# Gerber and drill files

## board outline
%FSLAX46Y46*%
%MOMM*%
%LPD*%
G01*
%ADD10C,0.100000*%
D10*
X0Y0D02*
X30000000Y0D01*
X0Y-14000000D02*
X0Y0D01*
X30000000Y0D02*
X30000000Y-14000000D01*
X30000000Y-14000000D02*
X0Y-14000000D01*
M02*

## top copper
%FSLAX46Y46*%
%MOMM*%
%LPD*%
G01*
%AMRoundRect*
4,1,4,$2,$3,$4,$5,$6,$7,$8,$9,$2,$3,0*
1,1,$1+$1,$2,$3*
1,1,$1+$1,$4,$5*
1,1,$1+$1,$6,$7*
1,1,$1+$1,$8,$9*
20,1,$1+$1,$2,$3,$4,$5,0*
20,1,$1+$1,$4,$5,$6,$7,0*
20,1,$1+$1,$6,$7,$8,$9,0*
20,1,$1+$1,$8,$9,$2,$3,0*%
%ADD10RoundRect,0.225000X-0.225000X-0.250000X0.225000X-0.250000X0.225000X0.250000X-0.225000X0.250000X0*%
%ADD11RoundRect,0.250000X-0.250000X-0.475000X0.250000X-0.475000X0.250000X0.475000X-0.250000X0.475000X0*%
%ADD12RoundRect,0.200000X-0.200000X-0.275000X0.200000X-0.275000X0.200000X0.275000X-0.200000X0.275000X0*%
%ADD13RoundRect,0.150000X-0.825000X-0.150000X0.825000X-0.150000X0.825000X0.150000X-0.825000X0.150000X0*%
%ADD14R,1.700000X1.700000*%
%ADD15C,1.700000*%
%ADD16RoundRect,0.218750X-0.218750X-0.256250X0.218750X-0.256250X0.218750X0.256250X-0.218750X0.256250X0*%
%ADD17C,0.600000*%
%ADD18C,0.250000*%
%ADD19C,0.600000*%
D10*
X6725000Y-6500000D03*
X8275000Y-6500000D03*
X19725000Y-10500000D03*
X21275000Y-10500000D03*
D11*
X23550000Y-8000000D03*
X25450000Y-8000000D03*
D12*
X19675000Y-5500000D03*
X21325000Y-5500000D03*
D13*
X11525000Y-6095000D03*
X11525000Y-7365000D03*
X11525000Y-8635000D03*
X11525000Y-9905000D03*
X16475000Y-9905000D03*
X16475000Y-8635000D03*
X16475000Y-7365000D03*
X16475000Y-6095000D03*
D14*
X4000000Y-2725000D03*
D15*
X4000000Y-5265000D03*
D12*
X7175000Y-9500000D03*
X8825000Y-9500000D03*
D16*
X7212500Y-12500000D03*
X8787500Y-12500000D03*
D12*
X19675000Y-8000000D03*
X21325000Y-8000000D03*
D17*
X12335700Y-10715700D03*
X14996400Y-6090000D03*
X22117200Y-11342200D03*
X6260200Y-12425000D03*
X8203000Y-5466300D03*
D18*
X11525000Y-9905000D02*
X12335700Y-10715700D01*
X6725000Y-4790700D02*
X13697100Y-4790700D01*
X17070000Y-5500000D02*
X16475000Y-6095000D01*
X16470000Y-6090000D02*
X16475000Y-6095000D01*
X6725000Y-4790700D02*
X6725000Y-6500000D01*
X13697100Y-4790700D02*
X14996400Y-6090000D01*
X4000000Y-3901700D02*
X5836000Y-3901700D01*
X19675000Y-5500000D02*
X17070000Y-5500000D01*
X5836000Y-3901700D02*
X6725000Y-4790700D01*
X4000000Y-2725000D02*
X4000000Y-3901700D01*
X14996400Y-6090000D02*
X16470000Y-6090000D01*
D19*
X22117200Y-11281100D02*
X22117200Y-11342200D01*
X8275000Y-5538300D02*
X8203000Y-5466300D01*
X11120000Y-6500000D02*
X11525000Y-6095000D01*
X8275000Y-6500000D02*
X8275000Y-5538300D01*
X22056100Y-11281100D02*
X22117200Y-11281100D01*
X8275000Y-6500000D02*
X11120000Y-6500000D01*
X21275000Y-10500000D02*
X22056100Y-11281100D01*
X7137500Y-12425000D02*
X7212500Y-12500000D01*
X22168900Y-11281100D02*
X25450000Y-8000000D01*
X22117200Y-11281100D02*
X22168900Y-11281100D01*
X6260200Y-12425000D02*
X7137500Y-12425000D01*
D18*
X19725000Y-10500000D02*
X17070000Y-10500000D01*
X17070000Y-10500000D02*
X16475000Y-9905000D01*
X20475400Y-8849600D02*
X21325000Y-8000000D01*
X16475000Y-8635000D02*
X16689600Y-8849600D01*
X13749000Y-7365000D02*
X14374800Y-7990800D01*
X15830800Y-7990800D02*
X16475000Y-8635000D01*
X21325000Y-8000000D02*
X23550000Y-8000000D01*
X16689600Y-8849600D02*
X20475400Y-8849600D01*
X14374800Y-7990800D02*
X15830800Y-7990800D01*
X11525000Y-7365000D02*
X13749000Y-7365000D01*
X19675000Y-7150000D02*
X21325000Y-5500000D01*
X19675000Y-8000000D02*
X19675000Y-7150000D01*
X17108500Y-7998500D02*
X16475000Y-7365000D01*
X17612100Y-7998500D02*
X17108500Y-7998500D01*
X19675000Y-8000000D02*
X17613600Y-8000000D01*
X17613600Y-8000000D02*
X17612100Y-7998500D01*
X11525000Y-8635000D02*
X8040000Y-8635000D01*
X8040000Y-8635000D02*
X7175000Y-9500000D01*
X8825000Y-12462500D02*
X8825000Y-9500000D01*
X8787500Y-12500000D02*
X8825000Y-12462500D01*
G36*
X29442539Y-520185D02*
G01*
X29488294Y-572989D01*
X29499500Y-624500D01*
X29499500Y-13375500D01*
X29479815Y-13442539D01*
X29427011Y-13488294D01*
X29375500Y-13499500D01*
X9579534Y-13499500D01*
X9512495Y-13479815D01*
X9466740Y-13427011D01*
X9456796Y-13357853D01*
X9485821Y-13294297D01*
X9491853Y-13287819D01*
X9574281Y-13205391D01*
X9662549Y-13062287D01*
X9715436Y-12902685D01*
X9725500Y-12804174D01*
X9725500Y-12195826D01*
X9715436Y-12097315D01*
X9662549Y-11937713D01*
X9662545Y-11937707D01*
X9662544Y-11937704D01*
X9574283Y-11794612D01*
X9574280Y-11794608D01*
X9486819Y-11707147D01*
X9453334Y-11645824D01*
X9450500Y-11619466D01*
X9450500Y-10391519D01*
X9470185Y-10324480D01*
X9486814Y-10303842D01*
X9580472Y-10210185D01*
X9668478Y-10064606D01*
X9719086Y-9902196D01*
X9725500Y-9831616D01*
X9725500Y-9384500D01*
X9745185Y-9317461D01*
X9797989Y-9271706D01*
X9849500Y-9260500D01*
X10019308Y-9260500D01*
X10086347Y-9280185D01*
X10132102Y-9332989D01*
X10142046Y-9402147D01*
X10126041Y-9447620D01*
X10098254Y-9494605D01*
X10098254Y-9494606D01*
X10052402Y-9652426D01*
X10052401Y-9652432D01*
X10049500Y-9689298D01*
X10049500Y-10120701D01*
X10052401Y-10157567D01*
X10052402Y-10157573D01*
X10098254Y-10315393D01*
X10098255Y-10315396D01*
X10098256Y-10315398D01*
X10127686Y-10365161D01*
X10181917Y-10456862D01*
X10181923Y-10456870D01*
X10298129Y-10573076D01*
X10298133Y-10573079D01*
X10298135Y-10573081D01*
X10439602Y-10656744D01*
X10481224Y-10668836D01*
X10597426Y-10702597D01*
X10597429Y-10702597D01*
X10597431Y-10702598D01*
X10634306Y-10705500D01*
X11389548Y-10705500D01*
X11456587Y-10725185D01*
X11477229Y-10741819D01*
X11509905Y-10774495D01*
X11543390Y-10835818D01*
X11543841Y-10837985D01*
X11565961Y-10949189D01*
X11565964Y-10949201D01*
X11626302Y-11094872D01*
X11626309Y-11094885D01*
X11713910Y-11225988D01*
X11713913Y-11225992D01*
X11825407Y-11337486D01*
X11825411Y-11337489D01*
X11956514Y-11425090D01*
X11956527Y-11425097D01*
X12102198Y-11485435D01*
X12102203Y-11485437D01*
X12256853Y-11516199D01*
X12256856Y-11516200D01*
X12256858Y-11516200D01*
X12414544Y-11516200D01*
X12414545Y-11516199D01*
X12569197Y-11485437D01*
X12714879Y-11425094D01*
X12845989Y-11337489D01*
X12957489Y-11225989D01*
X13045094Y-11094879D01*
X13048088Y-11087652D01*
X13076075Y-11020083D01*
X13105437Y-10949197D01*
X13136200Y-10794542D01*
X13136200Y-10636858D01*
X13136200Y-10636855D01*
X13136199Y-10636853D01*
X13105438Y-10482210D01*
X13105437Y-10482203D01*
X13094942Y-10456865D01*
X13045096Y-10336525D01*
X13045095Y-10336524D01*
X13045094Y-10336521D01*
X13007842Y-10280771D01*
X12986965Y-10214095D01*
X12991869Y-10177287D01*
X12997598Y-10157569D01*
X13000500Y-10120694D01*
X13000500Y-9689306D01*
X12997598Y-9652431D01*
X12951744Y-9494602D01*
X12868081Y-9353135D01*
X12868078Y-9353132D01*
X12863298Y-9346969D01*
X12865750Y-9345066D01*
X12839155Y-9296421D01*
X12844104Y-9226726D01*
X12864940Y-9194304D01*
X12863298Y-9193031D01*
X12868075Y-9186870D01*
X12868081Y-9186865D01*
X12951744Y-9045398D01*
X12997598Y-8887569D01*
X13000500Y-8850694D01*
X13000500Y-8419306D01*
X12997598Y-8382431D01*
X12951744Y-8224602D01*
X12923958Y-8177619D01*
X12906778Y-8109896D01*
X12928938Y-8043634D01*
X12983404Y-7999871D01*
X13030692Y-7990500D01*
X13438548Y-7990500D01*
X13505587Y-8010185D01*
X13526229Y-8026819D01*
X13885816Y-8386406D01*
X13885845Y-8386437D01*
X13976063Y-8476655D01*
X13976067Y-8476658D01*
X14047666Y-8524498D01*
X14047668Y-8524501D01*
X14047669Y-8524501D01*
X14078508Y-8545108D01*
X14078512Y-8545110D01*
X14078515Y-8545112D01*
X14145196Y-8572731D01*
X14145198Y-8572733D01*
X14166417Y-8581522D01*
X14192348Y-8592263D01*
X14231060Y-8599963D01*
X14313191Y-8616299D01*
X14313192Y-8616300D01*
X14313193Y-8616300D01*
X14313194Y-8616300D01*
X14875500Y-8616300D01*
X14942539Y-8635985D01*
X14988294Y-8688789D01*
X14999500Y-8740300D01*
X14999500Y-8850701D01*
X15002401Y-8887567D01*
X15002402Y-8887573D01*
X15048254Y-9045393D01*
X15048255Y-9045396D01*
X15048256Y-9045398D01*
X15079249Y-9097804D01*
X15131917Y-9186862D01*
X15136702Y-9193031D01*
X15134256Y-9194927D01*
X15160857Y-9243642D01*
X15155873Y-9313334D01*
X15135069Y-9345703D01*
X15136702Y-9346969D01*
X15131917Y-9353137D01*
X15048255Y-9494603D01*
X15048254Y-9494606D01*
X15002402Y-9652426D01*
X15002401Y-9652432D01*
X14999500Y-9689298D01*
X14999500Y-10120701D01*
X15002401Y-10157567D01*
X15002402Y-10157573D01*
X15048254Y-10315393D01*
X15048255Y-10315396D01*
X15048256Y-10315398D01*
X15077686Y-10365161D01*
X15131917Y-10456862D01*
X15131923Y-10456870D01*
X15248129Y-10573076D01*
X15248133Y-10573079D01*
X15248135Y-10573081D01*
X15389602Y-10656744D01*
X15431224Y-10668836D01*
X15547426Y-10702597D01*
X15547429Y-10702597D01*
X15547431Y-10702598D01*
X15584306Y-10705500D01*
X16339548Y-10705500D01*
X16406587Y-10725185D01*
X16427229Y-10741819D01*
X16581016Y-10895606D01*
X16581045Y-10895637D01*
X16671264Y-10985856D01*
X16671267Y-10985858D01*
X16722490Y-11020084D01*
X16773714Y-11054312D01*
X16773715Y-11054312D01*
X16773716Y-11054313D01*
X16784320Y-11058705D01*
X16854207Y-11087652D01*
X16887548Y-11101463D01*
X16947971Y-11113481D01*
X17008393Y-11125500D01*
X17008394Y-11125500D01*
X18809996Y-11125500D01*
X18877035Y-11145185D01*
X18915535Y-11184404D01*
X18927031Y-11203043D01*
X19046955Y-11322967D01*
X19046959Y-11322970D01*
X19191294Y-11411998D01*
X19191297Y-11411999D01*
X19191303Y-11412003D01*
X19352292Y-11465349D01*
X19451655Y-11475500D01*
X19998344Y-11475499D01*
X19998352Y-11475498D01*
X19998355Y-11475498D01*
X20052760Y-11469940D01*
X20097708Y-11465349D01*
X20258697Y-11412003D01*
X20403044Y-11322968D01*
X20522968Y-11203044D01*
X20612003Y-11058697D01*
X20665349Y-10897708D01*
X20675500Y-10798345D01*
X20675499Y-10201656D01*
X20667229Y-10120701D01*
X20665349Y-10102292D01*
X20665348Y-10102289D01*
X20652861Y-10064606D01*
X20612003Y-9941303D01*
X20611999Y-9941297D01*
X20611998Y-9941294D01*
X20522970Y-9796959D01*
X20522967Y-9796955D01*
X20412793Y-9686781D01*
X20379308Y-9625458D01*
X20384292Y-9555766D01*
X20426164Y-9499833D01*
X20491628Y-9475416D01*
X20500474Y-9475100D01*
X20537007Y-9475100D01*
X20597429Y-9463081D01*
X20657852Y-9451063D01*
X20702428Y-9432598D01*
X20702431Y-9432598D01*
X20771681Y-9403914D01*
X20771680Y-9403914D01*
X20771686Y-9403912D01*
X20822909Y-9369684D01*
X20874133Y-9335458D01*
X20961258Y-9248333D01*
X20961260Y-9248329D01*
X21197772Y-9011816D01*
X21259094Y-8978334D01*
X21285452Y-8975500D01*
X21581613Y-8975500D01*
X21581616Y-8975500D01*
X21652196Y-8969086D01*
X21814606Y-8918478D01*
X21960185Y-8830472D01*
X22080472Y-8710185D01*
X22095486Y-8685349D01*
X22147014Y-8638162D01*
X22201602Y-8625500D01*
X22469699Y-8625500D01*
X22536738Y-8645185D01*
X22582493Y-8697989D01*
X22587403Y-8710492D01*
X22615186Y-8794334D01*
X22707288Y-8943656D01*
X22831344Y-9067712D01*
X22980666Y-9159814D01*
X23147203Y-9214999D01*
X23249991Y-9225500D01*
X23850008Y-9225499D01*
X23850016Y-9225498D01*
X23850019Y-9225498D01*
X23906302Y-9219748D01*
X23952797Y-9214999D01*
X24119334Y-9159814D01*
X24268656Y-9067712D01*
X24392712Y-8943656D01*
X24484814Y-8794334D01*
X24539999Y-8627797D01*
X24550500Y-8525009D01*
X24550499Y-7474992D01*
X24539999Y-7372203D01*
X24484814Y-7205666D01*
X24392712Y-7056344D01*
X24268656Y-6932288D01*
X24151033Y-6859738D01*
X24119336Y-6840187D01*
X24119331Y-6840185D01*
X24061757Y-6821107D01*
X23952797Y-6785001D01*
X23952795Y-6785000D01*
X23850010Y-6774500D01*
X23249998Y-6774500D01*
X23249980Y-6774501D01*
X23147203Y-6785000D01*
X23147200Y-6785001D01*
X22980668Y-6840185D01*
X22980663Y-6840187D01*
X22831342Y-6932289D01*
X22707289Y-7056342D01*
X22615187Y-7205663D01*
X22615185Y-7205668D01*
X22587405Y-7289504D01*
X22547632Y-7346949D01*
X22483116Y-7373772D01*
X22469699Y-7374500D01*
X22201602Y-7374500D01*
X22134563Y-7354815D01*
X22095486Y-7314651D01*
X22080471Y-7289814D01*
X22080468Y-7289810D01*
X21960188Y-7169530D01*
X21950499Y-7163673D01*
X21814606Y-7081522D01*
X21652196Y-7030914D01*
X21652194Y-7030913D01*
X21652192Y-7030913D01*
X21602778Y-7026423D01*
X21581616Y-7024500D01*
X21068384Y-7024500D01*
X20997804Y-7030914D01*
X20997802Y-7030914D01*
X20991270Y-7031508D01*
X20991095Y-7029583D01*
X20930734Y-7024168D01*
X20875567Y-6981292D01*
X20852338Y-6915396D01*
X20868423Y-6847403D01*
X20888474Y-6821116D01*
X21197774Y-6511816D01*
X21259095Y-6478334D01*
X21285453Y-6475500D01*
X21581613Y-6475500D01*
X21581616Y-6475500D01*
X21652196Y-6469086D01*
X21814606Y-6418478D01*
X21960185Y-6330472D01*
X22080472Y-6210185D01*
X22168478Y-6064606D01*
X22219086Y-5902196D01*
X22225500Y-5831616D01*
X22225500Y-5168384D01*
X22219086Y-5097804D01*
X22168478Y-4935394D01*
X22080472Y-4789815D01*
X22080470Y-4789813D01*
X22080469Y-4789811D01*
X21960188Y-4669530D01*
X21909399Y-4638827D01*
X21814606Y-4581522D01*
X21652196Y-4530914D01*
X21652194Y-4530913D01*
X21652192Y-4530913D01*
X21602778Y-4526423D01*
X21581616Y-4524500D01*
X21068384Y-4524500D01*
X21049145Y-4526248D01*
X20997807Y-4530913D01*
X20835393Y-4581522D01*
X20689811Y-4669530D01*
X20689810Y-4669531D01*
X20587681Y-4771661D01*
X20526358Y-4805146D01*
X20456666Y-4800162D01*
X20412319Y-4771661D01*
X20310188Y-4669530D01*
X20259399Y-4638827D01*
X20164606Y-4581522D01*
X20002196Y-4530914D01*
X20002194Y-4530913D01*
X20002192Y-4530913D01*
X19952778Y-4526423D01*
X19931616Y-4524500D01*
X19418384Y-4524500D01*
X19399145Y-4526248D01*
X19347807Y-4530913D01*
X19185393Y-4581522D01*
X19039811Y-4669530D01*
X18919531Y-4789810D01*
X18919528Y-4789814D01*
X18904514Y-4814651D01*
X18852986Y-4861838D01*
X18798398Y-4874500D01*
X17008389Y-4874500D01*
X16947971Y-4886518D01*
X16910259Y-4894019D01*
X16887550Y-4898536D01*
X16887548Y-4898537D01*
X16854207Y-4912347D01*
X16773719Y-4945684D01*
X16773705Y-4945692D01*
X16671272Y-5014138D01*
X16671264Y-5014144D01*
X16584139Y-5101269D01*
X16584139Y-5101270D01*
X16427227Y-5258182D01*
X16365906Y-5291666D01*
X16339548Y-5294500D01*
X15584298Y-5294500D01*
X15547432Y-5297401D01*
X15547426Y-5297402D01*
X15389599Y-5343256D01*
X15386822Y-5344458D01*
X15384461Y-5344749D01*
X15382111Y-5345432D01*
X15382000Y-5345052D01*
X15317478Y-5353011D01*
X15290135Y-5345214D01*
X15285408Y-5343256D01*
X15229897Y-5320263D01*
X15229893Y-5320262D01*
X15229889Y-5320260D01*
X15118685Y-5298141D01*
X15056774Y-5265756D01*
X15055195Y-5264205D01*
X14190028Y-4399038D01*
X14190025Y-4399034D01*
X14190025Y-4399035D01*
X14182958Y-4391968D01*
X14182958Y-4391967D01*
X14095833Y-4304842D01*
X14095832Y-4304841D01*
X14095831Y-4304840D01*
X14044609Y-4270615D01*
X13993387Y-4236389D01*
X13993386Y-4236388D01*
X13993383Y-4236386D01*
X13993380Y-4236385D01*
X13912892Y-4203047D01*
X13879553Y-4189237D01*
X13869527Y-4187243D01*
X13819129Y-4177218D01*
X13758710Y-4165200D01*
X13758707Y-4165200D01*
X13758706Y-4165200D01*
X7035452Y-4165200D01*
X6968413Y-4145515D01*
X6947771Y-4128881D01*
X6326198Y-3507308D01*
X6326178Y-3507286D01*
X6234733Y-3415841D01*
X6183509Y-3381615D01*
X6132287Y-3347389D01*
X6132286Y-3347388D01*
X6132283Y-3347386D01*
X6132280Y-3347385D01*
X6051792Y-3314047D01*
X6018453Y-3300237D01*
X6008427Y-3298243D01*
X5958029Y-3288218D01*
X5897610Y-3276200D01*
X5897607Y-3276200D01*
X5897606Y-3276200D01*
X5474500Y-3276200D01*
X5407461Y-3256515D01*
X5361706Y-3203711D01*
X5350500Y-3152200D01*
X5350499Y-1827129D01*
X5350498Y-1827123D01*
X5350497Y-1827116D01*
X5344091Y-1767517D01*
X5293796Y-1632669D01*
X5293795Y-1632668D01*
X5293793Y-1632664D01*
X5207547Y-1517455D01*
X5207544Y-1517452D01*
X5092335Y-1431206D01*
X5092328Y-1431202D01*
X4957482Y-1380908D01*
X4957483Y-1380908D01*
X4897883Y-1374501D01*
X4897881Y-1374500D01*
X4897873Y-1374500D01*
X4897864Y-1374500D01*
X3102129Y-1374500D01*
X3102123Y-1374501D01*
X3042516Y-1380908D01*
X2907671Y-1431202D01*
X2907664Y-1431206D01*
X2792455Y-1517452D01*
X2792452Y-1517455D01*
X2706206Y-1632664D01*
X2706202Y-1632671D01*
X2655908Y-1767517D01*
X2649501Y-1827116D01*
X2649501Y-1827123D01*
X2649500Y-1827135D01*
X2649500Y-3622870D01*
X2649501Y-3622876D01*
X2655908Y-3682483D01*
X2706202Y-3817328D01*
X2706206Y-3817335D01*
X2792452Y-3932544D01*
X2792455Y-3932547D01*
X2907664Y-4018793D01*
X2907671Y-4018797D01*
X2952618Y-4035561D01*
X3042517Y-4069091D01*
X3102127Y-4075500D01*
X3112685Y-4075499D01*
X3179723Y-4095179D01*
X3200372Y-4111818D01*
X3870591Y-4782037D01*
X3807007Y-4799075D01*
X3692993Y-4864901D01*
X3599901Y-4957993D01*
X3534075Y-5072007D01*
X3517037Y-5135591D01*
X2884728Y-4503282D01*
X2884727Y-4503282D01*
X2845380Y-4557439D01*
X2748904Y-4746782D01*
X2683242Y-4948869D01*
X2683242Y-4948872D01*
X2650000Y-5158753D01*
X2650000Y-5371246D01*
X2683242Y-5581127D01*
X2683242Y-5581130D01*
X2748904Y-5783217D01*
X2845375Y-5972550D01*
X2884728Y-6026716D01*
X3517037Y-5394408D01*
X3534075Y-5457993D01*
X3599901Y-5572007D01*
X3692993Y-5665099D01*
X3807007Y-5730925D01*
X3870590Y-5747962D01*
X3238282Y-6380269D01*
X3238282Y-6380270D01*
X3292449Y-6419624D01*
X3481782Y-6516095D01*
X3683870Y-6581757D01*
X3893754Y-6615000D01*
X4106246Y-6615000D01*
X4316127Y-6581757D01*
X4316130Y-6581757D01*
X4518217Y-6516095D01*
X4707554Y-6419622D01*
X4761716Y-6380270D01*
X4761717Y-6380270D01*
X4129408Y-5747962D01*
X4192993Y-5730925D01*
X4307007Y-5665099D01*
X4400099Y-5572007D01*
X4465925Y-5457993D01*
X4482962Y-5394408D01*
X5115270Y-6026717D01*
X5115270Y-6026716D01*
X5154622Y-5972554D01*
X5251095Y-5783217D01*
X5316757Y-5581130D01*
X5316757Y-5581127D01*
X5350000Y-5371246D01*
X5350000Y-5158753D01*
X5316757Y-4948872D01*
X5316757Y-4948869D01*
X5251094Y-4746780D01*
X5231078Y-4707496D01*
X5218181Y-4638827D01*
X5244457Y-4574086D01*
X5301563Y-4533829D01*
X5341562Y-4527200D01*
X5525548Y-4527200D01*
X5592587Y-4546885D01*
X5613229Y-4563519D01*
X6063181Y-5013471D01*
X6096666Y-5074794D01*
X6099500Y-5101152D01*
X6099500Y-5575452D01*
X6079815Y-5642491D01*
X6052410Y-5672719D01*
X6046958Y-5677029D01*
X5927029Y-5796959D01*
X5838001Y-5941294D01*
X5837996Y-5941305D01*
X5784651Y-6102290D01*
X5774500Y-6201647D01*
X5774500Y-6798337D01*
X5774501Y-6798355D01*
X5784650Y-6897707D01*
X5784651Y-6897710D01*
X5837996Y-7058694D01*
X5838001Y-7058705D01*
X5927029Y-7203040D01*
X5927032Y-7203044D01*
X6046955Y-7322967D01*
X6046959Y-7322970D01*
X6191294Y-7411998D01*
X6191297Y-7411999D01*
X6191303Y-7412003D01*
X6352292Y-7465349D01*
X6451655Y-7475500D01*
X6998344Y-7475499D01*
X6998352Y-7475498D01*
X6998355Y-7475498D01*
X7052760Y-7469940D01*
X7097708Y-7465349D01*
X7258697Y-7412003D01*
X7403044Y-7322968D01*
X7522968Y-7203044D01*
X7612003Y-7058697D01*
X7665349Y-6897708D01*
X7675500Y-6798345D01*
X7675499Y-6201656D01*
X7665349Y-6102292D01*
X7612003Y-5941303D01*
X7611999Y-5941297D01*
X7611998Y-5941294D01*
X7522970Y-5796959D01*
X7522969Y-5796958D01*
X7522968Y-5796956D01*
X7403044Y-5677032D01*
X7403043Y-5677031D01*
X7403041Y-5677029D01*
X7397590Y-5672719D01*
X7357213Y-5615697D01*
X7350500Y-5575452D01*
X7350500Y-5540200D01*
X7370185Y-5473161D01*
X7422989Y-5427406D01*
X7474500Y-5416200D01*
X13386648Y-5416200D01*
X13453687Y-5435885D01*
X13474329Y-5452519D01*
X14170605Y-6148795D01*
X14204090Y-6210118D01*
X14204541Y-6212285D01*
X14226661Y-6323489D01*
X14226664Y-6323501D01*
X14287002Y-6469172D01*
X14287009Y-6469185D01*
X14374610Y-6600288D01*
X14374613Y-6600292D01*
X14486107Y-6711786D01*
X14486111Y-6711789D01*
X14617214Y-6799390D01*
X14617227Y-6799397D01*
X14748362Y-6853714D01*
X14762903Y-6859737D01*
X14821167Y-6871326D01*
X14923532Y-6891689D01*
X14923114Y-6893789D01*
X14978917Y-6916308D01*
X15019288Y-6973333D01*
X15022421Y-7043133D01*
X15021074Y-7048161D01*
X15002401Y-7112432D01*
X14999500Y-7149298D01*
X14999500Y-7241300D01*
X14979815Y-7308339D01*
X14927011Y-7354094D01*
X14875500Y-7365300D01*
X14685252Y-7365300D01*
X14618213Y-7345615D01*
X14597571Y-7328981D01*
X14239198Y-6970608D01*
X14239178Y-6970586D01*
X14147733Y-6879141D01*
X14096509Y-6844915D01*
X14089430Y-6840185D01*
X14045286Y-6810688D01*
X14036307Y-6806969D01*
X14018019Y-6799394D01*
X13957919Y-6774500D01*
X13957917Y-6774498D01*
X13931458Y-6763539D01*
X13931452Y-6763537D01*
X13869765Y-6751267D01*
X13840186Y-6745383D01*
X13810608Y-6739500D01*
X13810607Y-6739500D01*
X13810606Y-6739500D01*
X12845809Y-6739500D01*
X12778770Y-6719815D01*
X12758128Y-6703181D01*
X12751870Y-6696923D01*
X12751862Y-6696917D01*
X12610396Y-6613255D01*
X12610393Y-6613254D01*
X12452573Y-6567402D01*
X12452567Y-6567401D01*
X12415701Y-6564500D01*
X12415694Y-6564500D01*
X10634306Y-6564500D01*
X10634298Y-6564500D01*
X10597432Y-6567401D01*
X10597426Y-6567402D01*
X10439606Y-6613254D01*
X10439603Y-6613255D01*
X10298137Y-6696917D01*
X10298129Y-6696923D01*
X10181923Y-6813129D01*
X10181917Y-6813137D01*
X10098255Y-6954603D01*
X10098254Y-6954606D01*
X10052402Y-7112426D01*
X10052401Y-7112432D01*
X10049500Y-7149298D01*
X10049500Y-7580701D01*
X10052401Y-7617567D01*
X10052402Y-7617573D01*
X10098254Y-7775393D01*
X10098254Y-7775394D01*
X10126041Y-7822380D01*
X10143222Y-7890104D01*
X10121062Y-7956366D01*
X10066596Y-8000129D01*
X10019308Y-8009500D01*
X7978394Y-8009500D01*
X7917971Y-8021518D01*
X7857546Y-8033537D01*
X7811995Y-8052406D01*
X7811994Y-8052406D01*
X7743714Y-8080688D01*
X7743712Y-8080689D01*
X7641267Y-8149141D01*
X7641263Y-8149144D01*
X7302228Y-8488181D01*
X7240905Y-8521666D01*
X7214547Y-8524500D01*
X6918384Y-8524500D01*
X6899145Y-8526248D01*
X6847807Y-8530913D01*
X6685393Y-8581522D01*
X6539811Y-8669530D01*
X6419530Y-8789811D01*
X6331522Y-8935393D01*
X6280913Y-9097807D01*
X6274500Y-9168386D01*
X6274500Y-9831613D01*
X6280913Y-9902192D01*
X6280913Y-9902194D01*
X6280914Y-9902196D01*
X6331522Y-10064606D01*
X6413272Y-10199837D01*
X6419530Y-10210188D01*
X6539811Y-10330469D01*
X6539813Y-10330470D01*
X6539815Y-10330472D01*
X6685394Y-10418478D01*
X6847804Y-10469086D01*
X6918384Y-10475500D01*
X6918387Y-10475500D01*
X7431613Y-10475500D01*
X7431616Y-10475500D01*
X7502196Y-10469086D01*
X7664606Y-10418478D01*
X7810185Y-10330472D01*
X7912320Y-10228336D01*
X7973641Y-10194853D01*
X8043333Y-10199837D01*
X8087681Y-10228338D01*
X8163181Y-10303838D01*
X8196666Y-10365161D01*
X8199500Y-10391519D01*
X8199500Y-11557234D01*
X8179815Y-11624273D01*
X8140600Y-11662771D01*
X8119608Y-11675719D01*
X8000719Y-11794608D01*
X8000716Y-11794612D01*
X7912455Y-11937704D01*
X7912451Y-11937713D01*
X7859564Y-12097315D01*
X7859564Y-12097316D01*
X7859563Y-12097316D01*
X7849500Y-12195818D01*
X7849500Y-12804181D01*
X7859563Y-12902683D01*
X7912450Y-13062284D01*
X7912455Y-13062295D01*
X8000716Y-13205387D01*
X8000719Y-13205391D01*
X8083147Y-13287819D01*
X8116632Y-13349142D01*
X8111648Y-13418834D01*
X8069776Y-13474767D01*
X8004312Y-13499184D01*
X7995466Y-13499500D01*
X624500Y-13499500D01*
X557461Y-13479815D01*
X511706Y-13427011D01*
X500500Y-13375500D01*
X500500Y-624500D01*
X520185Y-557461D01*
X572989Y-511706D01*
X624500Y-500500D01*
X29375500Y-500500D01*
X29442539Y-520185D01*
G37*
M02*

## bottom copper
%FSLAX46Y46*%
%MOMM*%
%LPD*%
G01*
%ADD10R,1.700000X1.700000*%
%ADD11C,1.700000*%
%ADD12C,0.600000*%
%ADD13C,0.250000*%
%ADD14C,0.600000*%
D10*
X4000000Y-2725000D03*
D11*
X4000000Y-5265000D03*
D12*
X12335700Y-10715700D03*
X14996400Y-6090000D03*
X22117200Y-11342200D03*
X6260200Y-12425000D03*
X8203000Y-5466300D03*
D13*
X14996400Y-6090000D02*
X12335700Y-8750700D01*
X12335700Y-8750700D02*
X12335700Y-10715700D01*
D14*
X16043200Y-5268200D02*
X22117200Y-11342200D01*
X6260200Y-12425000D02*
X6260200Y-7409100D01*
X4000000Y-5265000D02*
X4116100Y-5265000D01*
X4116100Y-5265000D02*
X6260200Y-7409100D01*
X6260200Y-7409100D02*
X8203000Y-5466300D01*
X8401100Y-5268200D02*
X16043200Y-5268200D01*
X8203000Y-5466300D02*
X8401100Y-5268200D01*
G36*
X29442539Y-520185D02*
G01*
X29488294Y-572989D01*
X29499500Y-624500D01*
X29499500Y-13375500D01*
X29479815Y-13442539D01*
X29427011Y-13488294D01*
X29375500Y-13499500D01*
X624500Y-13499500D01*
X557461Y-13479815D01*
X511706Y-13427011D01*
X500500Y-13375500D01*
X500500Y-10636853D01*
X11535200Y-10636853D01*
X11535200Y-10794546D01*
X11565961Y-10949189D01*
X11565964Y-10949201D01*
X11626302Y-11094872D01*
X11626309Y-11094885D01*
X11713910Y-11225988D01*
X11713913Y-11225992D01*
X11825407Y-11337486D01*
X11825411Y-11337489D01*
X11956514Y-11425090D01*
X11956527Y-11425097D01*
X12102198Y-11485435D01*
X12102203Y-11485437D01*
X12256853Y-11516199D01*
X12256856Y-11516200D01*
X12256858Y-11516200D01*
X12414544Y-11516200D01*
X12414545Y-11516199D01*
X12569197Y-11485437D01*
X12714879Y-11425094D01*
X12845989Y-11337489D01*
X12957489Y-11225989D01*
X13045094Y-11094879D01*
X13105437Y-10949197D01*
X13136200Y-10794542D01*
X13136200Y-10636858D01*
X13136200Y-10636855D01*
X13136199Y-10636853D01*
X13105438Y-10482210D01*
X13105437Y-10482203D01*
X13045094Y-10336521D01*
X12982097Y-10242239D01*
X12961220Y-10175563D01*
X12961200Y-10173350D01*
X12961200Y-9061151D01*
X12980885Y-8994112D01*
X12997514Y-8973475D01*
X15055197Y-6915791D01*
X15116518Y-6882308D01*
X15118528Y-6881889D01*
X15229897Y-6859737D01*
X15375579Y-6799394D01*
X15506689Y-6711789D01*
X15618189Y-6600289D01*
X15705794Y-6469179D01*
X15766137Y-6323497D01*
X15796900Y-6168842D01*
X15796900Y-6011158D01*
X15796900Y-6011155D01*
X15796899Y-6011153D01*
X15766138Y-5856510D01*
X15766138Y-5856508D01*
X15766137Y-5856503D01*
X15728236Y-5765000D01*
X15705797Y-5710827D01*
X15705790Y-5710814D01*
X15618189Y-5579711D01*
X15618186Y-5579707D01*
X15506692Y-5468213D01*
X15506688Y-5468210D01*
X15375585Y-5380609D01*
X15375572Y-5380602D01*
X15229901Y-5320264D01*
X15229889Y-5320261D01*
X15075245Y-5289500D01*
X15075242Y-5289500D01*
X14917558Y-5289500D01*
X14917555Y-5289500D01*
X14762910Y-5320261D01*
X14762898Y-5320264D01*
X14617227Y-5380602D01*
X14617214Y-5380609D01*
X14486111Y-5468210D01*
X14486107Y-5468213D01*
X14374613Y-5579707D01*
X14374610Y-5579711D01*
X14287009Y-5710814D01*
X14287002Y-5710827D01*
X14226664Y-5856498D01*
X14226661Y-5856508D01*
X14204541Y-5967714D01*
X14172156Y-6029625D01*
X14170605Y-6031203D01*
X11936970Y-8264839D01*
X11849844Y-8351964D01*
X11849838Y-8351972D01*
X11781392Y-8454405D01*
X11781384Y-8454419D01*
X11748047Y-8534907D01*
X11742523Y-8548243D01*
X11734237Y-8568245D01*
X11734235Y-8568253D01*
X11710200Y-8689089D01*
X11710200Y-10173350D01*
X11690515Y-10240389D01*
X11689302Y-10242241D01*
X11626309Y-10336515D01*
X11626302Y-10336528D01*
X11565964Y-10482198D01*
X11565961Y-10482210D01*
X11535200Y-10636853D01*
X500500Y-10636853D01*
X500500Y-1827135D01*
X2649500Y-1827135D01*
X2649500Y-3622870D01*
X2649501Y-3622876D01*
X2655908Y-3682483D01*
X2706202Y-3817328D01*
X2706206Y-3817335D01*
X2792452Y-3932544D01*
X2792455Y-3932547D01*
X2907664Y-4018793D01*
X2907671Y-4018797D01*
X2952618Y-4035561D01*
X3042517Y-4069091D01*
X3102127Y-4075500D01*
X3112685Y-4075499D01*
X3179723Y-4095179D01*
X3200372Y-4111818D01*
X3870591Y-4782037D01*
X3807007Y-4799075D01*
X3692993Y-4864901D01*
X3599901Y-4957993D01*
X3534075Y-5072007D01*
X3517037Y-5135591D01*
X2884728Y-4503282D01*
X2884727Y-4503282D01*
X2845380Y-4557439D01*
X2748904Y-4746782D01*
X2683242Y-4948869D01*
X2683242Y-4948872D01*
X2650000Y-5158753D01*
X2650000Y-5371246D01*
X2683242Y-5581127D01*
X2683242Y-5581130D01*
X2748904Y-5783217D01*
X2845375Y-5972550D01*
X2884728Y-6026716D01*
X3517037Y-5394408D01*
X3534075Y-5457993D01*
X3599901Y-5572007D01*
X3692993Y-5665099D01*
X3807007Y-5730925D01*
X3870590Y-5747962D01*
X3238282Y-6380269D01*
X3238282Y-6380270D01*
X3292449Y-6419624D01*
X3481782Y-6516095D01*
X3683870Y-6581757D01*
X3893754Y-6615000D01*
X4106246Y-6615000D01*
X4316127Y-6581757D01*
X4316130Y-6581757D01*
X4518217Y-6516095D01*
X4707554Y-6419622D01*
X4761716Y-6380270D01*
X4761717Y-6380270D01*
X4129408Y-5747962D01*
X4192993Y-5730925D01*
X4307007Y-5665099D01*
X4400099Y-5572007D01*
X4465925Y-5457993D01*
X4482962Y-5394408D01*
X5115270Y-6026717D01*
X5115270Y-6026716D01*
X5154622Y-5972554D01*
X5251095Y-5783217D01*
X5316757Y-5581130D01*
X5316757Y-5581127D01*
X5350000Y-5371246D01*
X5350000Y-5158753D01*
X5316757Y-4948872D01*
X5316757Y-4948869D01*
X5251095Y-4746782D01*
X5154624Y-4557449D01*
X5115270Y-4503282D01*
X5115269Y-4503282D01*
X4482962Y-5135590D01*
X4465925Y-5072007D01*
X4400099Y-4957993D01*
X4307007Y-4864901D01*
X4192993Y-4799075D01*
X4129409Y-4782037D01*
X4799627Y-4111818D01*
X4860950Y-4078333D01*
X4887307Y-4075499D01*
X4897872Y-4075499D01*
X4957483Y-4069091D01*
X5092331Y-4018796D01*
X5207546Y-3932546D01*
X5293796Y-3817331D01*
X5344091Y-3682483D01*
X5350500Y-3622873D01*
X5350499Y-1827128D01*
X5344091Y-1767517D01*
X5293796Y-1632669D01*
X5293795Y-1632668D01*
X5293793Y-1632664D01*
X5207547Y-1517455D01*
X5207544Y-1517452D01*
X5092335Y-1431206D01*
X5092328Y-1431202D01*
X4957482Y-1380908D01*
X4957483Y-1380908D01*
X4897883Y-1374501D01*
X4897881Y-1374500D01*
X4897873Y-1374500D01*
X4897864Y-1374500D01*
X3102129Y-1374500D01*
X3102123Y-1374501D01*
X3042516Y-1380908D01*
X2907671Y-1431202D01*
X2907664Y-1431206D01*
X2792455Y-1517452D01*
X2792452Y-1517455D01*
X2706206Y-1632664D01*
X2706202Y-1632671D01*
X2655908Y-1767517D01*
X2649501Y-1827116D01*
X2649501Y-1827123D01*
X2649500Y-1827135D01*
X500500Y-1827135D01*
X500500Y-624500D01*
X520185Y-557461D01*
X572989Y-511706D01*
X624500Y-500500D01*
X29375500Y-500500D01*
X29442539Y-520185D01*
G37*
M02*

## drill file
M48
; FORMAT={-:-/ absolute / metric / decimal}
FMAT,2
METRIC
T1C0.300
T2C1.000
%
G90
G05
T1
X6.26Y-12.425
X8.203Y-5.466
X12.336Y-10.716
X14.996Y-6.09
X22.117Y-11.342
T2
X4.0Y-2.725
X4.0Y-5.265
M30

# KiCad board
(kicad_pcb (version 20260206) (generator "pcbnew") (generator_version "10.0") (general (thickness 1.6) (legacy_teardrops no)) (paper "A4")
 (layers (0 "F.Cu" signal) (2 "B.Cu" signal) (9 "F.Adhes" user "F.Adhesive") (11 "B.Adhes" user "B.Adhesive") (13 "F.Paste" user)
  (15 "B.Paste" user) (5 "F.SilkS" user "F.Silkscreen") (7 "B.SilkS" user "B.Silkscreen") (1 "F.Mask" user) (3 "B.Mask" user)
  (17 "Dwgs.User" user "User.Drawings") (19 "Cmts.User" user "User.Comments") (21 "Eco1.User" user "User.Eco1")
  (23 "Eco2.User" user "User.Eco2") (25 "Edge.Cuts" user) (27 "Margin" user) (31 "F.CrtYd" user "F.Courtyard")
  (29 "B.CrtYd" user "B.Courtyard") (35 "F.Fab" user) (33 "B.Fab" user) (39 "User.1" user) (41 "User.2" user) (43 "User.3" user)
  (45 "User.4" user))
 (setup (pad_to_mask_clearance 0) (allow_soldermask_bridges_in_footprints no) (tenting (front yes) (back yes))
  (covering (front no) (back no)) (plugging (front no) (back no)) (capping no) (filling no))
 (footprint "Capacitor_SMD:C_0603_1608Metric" (layer "F.Cu") (at 7.5 6.5)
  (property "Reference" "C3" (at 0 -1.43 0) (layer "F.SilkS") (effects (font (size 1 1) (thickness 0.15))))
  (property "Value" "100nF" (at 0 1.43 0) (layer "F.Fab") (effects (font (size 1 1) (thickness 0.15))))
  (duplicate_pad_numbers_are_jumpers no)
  (pad "1" smd roundrect (at -0.775 0) (size 0.9 0.95) (layers "F.Cu" "F.Mask" "F.Paste") (roundrect_rratio 0.25) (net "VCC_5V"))
  (pad "2" smd roundrect (at 0.775 0) (size 0.9 0.95) (layers "F.Cu" "F.Mask" "F.Paste") (roundrect_rratio 0.25) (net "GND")
   (zone_connect 2)))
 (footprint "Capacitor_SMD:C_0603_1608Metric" (layer "F.Cu") (at 20.5 10.5)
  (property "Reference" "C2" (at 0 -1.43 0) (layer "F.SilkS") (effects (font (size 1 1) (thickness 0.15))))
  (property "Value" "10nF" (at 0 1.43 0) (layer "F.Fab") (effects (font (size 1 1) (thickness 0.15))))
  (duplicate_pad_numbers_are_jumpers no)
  (pad "1" smd roundrect (at -0.775 0) (size 0.9 0.95) (layers "F.Cu" "F.Mask" "F.Paste") (roundrect_rratio 0.25) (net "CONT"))
  (pad "2" smd roundrect (at 0.775 0) (size 0.9 0.95) (layers "F.Cu" "F.Mask" "F.Paste") (roundrect_rratio 0.25) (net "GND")
   (zone_connect 2)))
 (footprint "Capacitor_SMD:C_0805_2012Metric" (layer "F.Cu") (at 24.5 8)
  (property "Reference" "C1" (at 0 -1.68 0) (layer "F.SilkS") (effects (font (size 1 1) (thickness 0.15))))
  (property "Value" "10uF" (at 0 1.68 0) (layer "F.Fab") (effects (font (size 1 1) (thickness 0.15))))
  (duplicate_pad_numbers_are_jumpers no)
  (pad "1" smd roundrect (at -0.95 0) (size 1 1.45) (layers "F.Cu" "F.Mask" "F.Paste") (roundrect_rratio 0.25) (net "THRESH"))
  (pad "2" smd roundrect (at 0.95 0) (size 1 1.45) (layers "F.Cu" "F.Mask" "F.Paste") (roundrect_rratio 0.25) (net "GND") (zone_connect 2)))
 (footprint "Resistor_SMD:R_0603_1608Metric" (layer "F.Cu") (at 20.5 5.5)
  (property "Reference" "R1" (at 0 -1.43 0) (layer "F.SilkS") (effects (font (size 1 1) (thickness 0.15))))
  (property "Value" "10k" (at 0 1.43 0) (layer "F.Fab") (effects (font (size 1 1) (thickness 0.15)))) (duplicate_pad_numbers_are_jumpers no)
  (pad "1" smd roundrect (at -0.825 0) (size 0.8 0.95) (layers "F.Cu" "F.Mask" "F.Paste") (roundrect_rratio 0.25) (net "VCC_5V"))
  (pad "2" smd roundrect (at 0.825 0) (size 0.8 0.95) (layers "F.Cu" "F.Mask" "F.Paste") (roundrect_rratio 0.25) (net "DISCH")))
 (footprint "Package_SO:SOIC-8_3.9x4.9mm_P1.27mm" (layer "F.Cu") (at 14 8)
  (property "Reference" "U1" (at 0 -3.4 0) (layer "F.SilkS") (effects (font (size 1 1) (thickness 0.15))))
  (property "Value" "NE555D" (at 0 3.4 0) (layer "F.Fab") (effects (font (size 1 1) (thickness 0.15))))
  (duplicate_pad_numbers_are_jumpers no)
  (pad "1" smd roundrect (at -2.475 -1.905) (size 1.95 0.6) (layers "F.Cu" "F.Mask" "F.Paste") (roundrect_rratio 0.25) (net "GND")
   (zone_connect 2))
  (pad "2" smd roundrect (at -2.475 -0.635) (size 1.95 0.6) (layers "F.Cu" "F.Mask" "F.Paste") (roundrect_rratio 0.25) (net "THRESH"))
  (pad "3" smd roundrect (at -2.475 0.635) (size 1.95 0.6) (layers "F.Cu" "F.Mask" "F.Paste") (roundrect_rratio 0.25) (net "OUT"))
  (pad "4" smd roundrect (at -2.475 1.905) (size 1.95 0.6) (layers "F.Cu" "F.Mask" "F.Paste") (roundrect_rratio 0.25) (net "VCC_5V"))
  (pad "5" smd roundrect (at 2.475 1.905) (size 1.95 0.6) (layers "F.Cu" "F.Mask" "F.Paste") (roundrect_rratio 0.25) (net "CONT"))
  (pad "6" smd roundrect (at 2.475 0.635) (size 1.95 0.6) (layers "F.Cu" "F.Mask" "F.Paste") (roundrect_rratio 0.25) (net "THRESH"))
  (pad "7" smd roundrect (at 2.475 -0.635) (size 1.95 0.6) (layers "F.Cu" "F.Mask" "F.Paste") (roundrect_rratio 0.25) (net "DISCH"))
  (pad "8" smd roundrect (at 2.475 -1.905) (size 1.95 0.6) (layers "F.Cu" "F.Mask" "F.Paste") (roundrect_rratio 0.25) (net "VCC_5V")))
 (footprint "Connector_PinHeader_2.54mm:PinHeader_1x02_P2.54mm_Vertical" (layer "F.Cu") (at 4 2.725)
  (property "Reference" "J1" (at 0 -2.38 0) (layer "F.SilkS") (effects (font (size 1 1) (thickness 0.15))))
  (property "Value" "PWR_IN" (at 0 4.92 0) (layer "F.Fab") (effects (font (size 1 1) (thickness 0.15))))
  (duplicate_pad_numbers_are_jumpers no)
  (pad "1" thru_hole rect (at 0 0) (size 1.7 1.7) (drill 1) (layers "*.Cu" "*.Mask") (remove_unused_layers no) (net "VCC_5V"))
  (pad "2" thru_hole circle (at 0 2.54) (size 1.7 1.7) (drill 1) (layers "*.Cu" "*.Mask") (remove_unused_layers no) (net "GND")))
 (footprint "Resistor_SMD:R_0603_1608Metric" (layer "F.Cu") (at 8 9.5)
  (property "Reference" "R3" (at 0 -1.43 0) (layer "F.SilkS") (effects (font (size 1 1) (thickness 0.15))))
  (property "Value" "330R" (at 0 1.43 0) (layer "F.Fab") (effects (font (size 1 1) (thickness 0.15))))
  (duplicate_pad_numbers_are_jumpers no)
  (pad "1" smd roundrect (at -0.825 0) (size 0.8 0.95) (layers "F.Cu" "F.Mask" "F.Paste") (roundrect_rratio 0.25) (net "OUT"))
  (pad "2" smd roundrect (at 0.825 0) (size 0.8 0.95) (layers "F.Cu" "F.Mask" "F.Paste") (roundrect_rratio 0.25) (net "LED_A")))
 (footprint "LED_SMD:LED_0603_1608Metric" (layer "F.Cu") (at 8 12.5)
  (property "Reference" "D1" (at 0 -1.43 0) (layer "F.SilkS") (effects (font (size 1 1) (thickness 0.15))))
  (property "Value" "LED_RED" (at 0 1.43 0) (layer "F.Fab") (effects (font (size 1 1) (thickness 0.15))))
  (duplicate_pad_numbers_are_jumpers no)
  (pad "1" smd roundrect (at -0.7875 0) (size 0.875 0.95) (layers "F.Cu" "F.Mask" "F.Paste") (roundrect_rratio 0.25) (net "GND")
   (zone_connect 2))
  (pad "2" smd roundrect (at 0.7875 0) (size 0.875 0.95) (layers "F.Cu" "F.Mask" "F.Paste") (roundrect_rratio 0.25) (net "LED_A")))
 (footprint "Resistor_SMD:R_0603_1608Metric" (layer "F.Cu") (at 20.5 8)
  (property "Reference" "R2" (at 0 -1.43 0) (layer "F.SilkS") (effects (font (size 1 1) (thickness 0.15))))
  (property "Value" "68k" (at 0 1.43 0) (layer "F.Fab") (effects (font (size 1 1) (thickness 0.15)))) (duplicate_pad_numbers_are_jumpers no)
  (pad "1" smd roundrect (at -0.825 0) (size 0.8 0.95) (layers "F.Cu" "F.Mask" "F.Paste") (roundrect_rratio 0.25) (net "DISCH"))
  (pad "2" smd roundrect (at 0.825 0) (size 0.8 0.95) (layers "F.Cu" "F.Mask" "F.Paste") (roundrect_rratio 0.25) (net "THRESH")))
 (gr_line (start 0 0) (end 30 0) (stroke (width 0.1) (type default)) (layer "Edge.Cuts"))
 (gr_line (start 0 14) (end 0 0) (stroke (width 0.1) (type default)) (layer "Edge.Cuts"))
 (gr_line (start 30 0) (end 30 14) (stroke (width 0.1) (type default)) (layer "Edge.Cuts"))
 (gr_line (start 30 14) (end 0 14) (stroke (width 0.1) (type default)) (layer "Edge.Cuts"))
 (segment (start 11.525 9.905) (end 12.3357 10.7157) (width 0.25) (layer "F.Cu") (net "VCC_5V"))
 (segment (start 6.725 4.7907) (end 13.6971 4.7907) (width 0.25) (layer "F.Cu") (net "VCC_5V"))
 (segment (start 17.07 5.5) (end 16.475 6.095) (width 0.25) (layer "F.Cu") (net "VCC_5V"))
 (segment (start 16.47 6.09) (end 16.475 6.095) (width 0.25) (layer "F.Cu") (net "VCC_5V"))
 (segment (start 6.725 4.7907) (end 6.725 6.5) (width 0.25) (layer "F.Cu") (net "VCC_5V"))
 (segment (start 13.6971 4.7907) (end 14.9964 6.09) (width 0.25) (layer "F.Cu") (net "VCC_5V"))
 (segment (start 4 3.9017) (end 5.836 3.9017) (width 0.25) (layer "F.Cu") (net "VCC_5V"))
 (segment (start 19.675 5.5) (end 17.07 5.5) (width 0.25) (layer "F.Cu") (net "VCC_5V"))
 (segment (start 5.836 3.9017) (end 6.725 4.7907) (width 0.25) (layer "F.Cu") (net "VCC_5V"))
 (segment (start 4 2.725) (end 4 3.9017) (width 0.25) (layer "F.Cu") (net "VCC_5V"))
 (segment (start 14.9964 6.09) (end 16.47 6.09) (width 0.25) (layer "F.Cu") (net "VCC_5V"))
 (via (at 12.3357 10.7157) (size 0.6) (drill 0.3) (layers "F.Cu" "B.Cu") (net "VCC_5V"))
 (via (at 14.9964 6.09) (size 0.6) (drill 0.3) (layers "F.Cu" "B.Cu") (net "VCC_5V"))
 (segment (start 14.9964 6.09) (end 12.3357 8.7507) (width 0.25) (layer "B.Cu") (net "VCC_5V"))
 (segment (start 12.3357 8.7507) (end 12.3357 10.7157) (width 0.25) (layer "B.Cu") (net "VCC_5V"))
 (segment (start 22.1172 11.2811) (end 22.1172 11.3422) (width 0.6) (layer "F.Cu") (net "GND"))
 (segment (start 8.275 5.5383) (end 8.203 5.4663) (width 0.6) (layer "F.Cu") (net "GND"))
 (segment (start 11.12 6.5) (end 11.525 6.095) (width 0.6) (layer "F.Cu") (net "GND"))
 (segment (start 8.275 6.5) (end 8.275 5.5383) (width 0.6) (layer "F.Cu") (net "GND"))
 (segment (start 22.0561 11.2811) (end 22.1172 11.2811) (width 0.6) (layer "F.Cu") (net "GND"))
 (segment (start 8.275 6.5) (end 11.12 6.5) (width 0.6) (layer "F.Cu") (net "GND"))
 (segment (start 21.275 10.5) (end 22.0561 11.2811) (width 0.6) (layer "F.Cu") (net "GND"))
 (segment (start 7.1375 12.425) (end 7.2125 12.5) (width 0.6) (layer "F.Cu") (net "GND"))
 (segment (start 22.1689 11.2811) (end 25.45 8) (width 0.6) (layer "F.Cu") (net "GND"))
 (segment (start 22.1172 11.2811) (end 22.1689 11.2811) (width 0.6) (layer "F.Cu") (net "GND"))
 (segment (start 6.2602 12.425) (end 7.1375 12.425) (width 0.6) (layer "F.Cu") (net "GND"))
 (via (at 22.1172 11.3422) (size 0.6) (drill 0.3) (layers "F.Cu" "B.Cu") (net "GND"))
 (via (at 6.2602 12.425) (size 0.6) (drill 0.3) (layers "F.Cu" "B.Cu") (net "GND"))
 (via (at 8.203 5.4663) (size 0.6) (drill 0.3) (layers "F.Cu" "B.Cu") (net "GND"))
 (segment (start 16.0432 5.2682) (end 22.1172 11.3422) (width 0.6) (layer "B.Cu") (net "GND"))
 (segment (start 6.2602 12.425) (end 6.2602 7.4091) (width 0.6) (layer "B.Cu") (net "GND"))
 (segment (start 4 5.265) (end 4.1161 5.265) (width 0.6) (layer "B.Cu") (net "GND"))
 (segment (start 4.1161 5.265) (end 6.2602 7.4091) (width 0.6) (layer "B.Cu") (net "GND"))
 (segment (start 6.2602 7.4091) (end 8.203 5.4663) (width 0.6) (layer "B.Cu") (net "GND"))
 (segment (start 8.4011 5.2682) (end 16.0432 5.2682) (width 0.6) (layer "B.Cu") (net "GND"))
 (segment (start 8.203 5.4663) (end 8.4011 5.2682) (width 0.6) (layer "B.Cu") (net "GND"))
 (segment (start 19.725 10.5) (end 17.07 10.5) (width 0.25) (layer "F.Cu") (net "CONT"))
 (segment (start 17.07 10.5) (end 16.475 9.905) (width 0.25) (layer "F.Cu") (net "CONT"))
 (segment (start 20.4754 8.8496) (end 21.325 8) (width 0.25) (layer "F.Cu") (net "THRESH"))
 (segment (start 16.475 8.635) (end 16.6896 8.8496) (width 0.25) (layer "F.Cu") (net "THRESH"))
 (segment (start 13.749 7.365) (end 14.3748 7.9908) (width 0.25) (layer "F.Cu") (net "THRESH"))
 (segment (start 15.8308 7.9908) (end 16.475 8.635) (width 0.25) (layer "F.Cu") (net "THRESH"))
 (segment (start 21.325 8) (end 23.55 8) (width 0.25) (layer "F.Cu") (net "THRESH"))
 (segment (start 16.6896 8.8496) (end 20.4754 8.8496) (width 0.25) (layer "F.Cu") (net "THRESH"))
 (segment (start 14.3748 7.9908) (end 15.8308 7.9908) (width 0.25) (layer "F.Cu") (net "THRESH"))
 (segment (start 11.525 7.365) (end 13.749 7.365) (width 0.25) (layer "F.Cu") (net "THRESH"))
 (segment (start 19.675 7.15) (end 21.325 5.5) (width 0.25) (layer "F.Cu") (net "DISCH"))
 (segment (start 19.675 8) (end 19.675 7.15) (width 0.25) (layer "F.Cu") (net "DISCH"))
 (segment (start 17.1085 7.9985) (end 16.475 7.365) (width 0.25) (layer "F.Cu") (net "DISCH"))
 (segment (start 17.6121 7.9985) (end 17.1085 7.9985) (width 0.25) (layer "F.Cu") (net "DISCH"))
 (segment (start 19.675 8) (end 17.6136 8) (width 0.25) (layer "F.Cu") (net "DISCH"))
 (segment (start 17.6136 8) (end 17.6121 7.9985) (width 0.25) (layer "F.Cu") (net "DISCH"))
 (segment (start 11.525 8.635) (end 8.04 8.635) (width 0.25) (layer "F.Cu") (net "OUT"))
 (segment (start 8.04 8.635) (end 7.175 9.5) (width 0.25) (layer "F.Cu") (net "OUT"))
 (segment (start 8.825 12.4625) (end 8.825 9.5) (width 0.25) (layer "F.Cu") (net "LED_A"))
 (segment (start 8.7875 12.5) (end 8.825 12.4625) (width 0.25) (layer "F.Cu") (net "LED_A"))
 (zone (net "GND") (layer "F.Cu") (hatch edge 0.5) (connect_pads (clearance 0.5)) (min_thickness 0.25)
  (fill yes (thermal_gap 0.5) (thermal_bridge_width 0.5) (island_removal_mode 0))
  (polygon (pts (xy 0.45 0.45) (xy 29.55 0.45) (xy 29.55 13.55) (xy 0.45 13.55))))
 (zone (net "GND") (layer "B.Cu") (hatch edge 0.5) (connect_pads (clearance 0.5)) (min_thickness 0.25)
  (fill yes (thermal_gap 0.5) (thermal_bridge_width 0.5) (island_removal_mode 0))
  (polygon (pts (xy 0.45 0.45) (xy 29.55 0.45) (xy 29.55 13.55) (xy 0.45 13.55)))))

